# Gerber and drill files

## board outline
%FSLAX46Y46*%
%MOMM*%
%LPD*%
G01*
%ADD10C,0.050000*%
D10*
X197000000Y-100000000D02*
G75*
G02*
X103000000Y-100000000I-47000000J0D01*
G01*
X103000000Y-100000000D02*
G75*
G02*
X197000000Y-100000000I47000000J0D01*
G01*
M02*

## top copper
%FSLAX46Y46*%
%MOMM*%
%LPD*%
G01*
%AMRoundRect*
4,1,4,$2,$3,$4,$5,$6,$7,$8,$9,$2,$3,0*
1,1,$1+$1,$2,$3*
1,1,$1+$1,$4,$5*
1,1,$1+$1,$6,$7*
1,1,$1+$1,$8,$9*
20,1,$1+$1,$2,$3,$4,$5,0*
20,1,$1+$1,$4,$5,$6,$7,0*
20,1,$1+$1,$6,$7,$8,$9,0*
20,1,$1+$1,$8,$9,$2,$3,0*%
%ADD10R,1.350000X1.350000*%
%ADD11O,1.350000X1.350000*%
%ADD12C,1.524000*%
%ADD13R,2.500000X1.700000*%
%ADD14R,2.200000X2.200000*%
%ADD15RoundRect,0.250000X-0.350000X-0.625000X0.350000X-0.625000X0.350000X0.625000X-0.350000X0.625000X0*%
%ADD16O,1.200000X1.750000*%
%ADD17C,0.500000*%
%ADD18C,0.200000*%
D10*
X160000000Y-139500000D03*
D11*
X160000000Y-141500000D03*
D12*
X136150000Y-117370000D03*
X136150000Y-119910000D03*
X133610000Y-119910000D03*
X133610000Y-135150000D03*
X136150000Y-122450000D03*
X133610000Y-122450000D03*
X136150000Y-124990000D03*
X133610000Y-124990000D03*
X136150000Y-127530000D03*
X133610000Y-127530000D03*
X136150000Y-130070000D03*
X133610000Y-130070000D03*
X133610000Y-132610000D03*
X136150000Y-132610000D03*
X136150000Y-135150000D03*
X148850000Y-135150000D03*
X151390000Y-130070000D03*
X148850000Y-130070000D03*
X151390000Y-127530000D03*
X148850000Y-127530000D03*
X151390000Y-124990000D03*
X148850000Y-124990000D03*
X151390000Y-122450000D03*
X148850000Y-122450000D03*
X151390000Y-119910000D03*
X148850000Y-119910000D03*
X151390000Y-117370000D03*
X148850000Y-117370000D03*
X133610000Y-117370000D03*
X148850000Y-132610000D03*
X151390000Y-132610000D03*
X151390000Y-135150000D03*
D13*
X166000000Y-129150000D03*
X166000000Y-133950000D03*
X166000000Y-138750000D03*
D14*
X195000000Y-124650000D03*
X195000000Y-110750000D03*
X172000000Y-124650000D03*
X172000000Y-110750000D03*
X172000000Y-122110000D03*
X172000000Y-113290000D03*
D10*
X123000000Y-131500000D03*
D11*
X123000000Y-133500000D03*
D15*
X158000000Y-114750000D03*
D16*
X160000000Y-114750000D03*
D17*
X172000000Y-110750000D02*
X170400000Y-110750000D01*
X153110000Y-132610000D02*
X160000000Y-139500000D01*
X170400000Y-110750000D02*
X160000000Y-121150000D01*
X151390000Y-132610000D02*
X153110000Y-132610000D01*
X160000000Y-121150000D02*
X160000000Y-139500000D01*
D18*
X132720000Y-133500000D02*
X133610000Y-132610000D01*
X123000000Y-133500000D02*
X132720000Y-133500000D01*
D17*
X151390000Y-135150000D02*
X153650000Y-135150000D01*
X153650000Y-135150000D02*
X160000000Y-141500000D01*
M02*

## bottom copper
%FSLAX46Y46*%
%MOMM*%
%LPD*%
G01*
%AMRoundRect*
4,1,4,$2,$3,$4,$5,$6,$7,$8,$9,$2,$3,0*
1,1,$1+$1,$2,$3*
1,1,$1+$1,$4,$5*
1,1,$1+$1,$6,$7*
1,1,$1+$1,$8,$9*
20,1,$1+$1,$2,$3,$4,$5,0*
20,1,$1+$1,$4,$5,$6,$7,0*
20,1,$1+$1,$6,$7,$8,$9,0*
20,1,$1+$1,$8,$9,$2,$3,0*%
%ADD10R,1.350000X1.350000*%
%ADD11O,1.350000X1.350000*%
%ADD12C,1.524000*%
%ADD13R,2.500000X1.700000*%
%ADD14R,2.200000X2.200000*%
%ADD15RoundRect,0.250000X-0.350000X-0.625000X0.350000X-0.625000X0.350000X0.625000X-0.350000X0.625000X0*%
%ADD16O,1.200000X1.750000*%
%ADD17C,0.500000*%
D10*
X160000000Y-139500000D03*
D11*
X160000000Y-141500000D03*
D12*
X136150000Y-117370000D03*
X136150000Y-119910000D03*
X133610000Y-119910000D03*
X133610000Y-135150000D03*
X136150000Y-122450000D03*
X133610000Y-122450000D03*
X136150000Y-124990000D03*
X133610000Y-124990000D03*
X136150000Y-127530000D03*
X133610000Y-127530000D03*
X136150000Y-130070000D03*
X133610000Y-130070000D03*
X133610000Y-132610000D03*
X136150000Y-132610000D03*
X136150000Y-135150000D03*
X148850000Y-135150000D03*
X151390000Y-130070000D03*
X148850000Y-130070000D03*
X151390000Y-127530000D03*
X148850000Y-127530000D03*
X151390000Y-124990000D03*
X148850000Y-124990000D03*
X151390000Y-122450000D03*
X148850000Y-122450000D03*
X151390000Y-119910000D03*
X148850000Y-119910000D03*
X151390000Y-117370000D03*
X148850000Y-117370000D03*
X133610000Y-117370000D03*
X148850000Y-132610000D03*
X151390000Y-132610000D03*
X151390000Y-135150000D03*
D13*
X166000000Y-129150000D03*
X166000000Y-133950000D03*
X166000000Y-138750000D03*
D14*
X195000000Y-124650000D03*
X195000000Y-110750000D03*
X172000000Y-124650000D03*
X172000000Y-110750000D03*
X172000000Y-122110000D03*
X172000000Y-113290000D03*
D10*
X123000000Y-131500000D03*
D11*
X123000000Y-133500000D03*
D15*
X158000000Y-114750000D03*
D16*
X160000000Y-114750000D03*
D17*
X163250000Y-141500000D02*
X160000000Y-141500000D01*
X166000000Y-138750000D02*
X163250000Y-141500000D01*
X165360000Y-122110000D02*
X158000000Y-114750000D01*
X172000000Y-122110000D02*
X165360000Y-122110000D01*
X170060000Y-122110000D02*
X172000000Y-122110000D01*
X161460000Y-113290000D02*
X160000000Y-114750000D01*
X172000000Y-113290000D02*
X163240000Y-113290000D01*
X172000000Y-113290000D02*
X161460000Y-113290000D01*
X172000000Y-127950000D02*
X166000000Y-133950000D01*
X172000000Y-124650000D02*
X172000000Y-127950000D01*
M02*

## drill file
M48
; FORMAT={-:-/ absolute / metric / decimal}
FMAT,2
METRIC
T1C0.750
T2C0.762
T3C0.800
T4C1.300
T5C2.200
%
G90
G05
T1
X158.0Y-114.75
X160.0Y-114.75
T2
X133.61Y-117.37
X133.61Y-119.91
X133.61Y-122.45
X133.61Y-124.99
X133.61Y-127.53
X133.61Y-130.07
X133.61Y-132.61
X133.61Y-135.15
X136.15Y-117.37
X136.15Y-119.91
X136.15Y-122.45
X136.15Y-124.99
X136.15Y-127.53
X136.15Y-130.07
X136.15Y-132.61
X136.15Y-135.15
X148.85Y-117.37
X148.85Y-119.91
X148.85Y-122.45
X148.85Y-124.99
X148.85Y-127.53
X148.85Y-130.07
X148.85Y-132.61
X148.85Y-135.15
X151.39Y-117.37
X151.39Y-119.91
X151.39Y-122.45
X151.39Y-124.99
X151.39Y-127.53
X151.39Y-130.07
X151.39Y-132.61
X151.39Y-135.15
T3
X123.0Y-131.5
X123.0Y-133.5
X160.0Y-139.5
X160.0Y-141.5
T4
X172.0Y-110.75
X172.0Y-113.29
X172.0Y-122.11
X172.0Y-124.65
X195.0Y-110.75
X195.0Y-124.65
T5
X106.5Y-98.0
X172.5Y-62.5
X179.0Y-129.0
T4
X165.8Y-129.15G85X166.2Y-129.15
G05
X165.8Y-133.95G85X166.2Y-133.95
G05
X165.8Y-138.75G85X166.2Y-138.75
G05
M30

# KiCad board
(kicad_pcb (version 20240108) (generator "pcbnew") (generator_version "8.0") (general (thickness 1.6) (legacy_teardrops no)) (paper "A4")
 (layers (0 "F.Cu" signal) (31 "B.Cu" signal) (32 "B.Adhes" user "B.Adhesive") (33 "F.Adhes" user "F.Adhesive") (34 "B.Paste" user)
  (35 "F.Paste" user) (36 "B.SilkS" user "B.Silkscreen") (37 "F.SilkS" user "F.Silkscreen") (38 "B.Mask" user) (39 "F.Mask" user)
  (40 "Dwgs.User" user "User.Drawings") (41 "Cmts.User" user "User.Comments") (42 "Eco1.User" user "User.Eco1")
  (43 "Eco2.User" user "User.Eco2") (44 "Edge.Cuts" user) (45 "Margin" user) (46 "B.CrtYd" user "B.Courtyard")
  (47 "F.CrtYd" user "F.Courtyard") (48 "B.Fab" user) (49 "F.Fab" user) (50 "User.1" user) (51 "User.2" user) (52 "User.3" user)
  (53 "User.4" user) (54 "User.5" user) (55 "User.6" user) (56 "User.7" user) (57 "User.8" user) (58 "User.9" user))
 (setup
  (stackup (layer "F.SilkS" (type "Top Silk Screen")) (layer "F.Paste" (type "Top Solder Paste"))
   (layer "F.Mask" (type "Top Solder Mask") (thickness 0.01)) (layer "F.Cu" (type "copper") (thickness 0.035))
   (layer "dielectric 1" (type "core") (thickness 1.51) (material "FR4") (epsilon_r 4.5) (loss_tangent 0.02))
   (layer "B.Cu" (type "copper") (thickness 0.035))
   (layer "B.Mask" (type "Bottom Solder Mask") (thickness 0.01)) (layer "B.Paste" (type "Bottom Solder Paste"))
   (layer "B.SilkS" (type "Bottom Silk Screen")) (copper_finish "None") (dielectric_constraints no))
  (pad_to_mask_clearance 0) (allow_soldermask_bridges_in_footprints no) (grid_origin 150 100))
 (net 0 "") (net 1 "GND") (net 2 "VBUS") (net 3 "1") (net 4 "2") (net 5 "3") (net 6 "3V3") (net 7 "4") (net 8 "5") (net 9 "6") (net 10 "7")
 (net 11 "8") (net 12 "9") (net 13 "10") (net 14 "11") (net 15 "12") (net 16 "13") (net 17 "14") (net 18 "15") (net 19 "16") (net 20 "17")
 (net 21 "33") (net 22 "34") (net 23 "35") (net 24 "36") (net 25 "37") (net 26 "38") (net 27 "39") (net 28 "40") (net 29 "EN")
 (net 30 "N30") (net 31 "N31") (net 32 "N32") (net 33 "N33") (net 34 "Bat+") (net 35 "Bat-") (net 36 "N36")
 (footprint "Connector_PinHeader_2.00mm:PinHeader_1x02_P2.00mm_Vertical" (layer "F.Cu") (at 160 139.5)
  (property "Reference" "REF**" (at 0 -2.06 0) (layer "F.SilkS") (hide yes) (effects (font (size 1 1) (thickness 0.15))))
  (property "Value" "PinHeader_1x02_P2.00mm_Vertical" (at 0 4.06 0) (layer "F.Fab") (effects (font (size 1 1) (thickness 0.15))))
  (pad "1" thru_hole rect (at 0 0) (size 1.35 1.35) (drill 0.8) (layers "*.Cu" "*.Mask") (remove_unused_layers no) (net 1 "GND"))
  (pad "2" thru_hole oval (at 0 2) (size 1.35 1.35) (drill 0.8) (layers "*.Cu" "*.Mask") (remove_unused_layers no) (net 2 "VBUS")))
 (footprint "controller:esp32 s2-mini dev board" (layer "F.Cu") (at 142.5 122.45)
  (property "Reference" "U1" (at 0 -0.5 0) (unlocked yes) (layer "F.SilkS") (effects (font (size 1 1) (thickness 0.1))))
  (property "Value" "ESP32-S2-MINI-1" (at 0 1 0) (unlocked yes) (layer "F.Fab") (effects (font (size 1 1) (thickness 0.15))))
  (pad "1" thru_hole circle (at -6.35 -5.08) (size 1.524 1.524) (drill 0.762) (layers "*.Cu" "*.Mask") (remove_unused_layers no) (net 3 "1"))
  (pad "2" thru_hole circle (at -6.35 -2.54) (size 1.524 1.524) (drill 0.762) (layers "*.Cu" "*.Mask") (remove_unused_layers no) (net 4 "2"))
  (pad "3" thru_hole circle (at -8.89 -2.54) (size 1.524 1.524) (drill 0.762) (layers "*.Cu" "*.Mask") (remove_unused_layers no) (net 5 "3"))
  (pad "3V3" thru_hole circle (at -8.89 12.7) (size 1.524 1.524) (drill 0.762) (layers "*.Cu" "*.Mask") (remove_unused_layers no)
   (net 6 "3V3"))
  (pad "4" thru_hole circle (at -6.35 0) (size 1.524 1.524) (drill 0.762) (layers "*.Cu" "*.Mask") (remove_unused_layers no) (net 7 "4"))
  (pad "5" thru_hole circle (at -8.89 0) (size 1.524 1.524) (drill 0.762) (layers "*.Cu" "*.Mask") (remove_unused_layers no) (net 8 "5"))
  (pad "6" thru_hole circle (at -6.35 2.54) (size 1.524 1.524) (drill 0.762) (layers "*.Cu" "*.Mask") (remove_unused_layers no) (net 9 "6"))
  (pad "7" thru_hole circle (at -8.89 2.54) (size 1.524 1.524) (drill 0.762) (layers "*.Cu" "*.Mask") (remove_unused_layers no) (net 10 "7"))
  (pad "8" thru_hole circle (at -6.35 5.08) (size 1.524 1.524) (drill 0.762) (layers "*.Cu" "*.Mask") (remove_unused_layers no) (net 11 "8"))
  (pad "9" thru_hole circle (at -8.89 5.08) (size 1.524 1.524) (drill 0.762) (layers "*.Cu" "*.Mask") (remove_unused_layers no) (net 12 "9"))
  (pad "10" thru_hole circle (at -6.35 7.62) (size 1.524 1.524) (drill 0.762) (layers "*.Cu" "*.Mask") (remove_unused_layers no)
   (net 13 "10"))
  (pad "11" thru_hole circle (at -8.89 7.62) (size 1.524 1.524) (drill 0.762) (layers "*.Cu" "*.Mask") (remove_unused_layers no)
   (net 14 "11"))
  (pad "12" thru_hole circle (at -8.89 10.16) (size 1.524 1.524) (drill 0.762) (layers "*.Cu" "*.Mask") (remove_unused_layers no)
   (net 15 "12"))
  (pad "13" thru_hole circle (at -6.35 10.16) (size 1.524 1.524) (drill 0.762) (layers "*.Cu" "*.Mask") (remove_unused_layers no)
   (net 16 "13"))
  (pad "14" thru_hole circle (at -6.35 12.7) (size 1.524 1.524) (drill 0.762) (layers "*.Cu" "*.Mask") (remove_unused_layers no)
   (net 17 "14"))
  (pad "15" thru_hole circle (at 6.35 12.7) (size 1.524 1.524) (drill 0.762) (layers "*.Cu" "*.Mask") (remove_unused_layers no)
   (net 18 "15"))
  (pad "16" thru_hole circle (at 8.89 7.62) (size 1.524 1.524) (drill 0.762) (layers "*.Cu" "*.Mask") (remove_unused_layers no)
   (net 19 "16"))
  (pad "17" thru_hole circle (at 6.35 7.62) (size 1.524 1.524) (drill 0.762) (layers "*.Cu" "*.Mask") (remove_unused_layers no))
  (pad "18" thru_hole circle (at 8.89 5.08) (size 1.524 1.524) (drill 0.762) (layers "*.Cu" "*.Mask") (remove_unused_layers no))
  (pad "21" thru_hole circle (at 6.35 5.08) (size 1.524 1.524) (drill 0.762) (layers "*.Cu" "*.Mask") (remove_unused_layers no)
   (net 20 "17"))
  (pad "33" thru_hole circle (at 8.89 2.54) (size 1.524 1.524) (drill 0.762) (layers "*.Cu" "*.Mask") (remove_unused_layers no)
   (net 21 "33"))
  (pad "34" thru_hole circle (at 6.35 2.54) (size 1.524 1.524) (drill 0.762) (layers "*.Cu" "*.Mask") (remove_unused_layers no)
   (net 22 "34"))
  (pad "35" thru_hole circle (at 8.89 0) (size 1.524 1.524) (drill 0.762) (layers "*.Cu" "*.Mask") (remove_unused_layers no) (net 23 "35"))
  (pad "36" thru_hole circle (at 6.35 0) (size 1.524 1.524) (drill 0.762) (layers "*.Cu" "*.Mask") (remove_unused_layers no) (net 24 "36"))
  (pad "37" thru_hole circle (at 8.89 -2.54) (size 1.524 1.524) (drill 0.762) (layers "*.Cu" "*.Mask") (remove_unused_layers no)
   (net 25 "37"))
  (pad "38" thru_hole circle (at 6.35 -2.54) (size 1.524 1.524) (drill 0.762) (layers "*.Cu" "*.Mask") (remove_unused_layers no)
   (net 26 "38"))
  (pad "39" thru_hole circle (at 8.89 -5.08) (size 1.524 1.524) (drill 0.762) (layers "*.Cu" "*.Mask") (remove_unused_layers no)
   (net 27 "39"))
  (pad "40" thru_hole circle (at 6.35 -5.08) (size 1.524 1.524) (drill 0.762) (layers "*.Cu" "*.Mask") (remove_unused_layers no)
   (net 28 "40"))
  (pad "EN" thru_hole circle (at -8.89 -5.08) (size 1.524 1.524) (drill 0.762) (layers "*.Cu" "*.Mask") (remove_unused_layers no)
   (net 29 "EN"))
  (pad "GND" thru_hole circle (at 6.35 10.16) (size 1.524 1.524) (drill 0.762) (layers "*.Cu" "*.Mask") (remove_unused_layers no)
   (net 1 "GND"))
  (pad "GND" thru_hole circle (at 8.89 10.16) (size 1.524 1.524) (drill 0.762) (layers "*.Cu" "*.Mask") (remove_unused_layers no)
   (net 1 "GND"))
  (pad "VBUS" thru_hole circle (at 8.89 12.7) (size 1.524 1.524) (drill 0.762) (layers "*.Cu" "*.Mask") (remove_unused_layers no)))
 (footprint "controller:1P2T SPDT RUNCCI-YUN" (layer "F.Cu") (at 166 133.95)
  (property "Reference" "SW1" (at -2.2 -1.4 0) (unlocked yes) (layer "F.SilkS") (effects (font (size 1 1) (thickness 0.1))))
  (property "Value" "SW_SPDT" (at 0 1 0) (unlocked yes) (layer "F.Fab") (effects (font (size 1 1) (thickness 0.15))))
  (pad "1" thru_hole rect (at 0 -4.8) (size 2.5 1.7) (drill oval 1.7 1.3) (layers "*.Cu" "*.Mask") (remove_unused_layers no) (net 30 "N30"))
  (pad "2" thru_hole rect (at 0 0) (size 2.5 1.7) (drill oval 1.7 1.3) (layers "*.Cu" "*.Mask") (remove_unused_layers no) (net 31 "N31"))
  (pad "3" thru_hole rect (at 0 4.8) (size 2.5 1.7) (drill oval 1.7 1.3) (layers "*.Cu" "*.Mask") (remove_unused_layers no) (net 2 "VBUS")))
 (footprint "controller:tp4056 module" (layer "F.Cu") (at 195 124.65 180)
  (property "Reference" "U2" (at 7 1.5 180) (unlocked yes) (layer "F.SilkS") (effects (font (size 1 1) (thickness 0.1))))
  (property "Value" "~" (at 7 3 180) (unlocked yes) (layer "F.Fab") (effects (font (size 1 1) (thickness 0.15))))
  (pad "1" thru_hole rect (at 0 0 180) (size 2.2 2.2) (drill 1.3) (layers "*.Cu" "*.Mask") (remove_unused_layers no) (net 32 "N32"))
  (pad "2" thru_hole rect (at 0 13.9 180) (size 2.2 2.2) (drill 1.3) (layers "*.Cu" "*.Mask") (remove_unused_layers no) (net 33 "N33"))
  (pad "3" thru_hole rect (at 23 0 180) (size 2.2 2.2) (drill 1.3) (layers "*.Cu" "*.Mask") (remove_unused_layers no) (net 31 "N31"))
  (pad "4" thru_hole rect (at 23 13.9 180) (size 2.2 2.2) (drill 1.3) (layers "*.Cu" "*.Mask") (remove_unused_layers no) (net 1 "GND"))
  (pad "5" thru_hole rect (at 23 2.54 180) (size 2.2 2.2) (drill 1.3) (layers "*.Cu" "*.Mask") (remove_unused_layers no) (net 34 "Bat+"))
  (pad "6" thru_hole rect (at 23 11.36 180) (size 2.2 2.2) (drill 1.3) (layers "*.Cu" "*.Mask") (remove_unused_layers no) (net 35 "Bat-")))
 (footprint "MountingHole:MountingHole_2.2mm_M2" (layer "F.Cu") (at 172.5 62.5)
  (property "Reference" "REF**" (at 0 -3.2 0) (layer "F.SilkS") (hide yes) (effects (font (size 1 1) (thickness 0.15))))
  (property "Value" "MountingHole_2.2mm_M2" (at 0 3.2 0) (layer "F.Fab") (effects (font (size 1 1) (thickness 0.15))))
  (pad "" np_thru_hole circle (at 0 0) (size 2.2 2.2) (drill 2.2) (layers "*.Cu" "*.Mask")))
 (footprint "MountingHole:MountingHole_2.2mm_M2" (layer "F.Cu") (at 179 129)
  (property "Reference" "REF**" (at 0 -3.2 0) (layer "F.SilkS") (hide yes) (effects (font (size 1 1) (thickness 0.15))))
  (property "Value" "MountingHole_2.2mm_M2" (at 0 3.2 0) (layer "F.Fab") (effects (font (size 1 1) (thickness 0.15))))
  (pad "" np_thru_hole circle (at 0 0) (size 2.2 2.2) (drill 2.2) (layers "F&B.Cu" "*.Mask")))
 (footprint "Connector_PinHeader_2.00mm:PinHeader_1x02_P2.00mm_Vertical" (layer "F.Cu") (at 123 131.5)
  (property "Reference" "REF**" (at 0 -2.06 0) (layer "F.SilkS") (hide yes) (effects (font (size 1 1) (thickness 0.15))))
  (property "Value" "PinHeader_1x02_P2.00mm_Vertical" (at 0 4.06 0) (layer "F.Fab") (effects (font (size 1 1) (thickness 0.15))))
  (pad "1" thru_hole rect (at 0 0) (size 1.35 1.35) (drill 0.8) (layers "*.Cu" "*.Mask") (remove_unused_layers no) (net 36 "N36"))
  (pad "2" thru_hole oval (at 0 2) (size 1.35 1.35) (drill 0.8) (layers "*.Cu" "*.Mask") (remove_unused_layers no) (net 15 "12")))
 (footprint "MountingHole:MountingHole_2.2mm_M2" (layer "F.Cu") (at 106.5 98)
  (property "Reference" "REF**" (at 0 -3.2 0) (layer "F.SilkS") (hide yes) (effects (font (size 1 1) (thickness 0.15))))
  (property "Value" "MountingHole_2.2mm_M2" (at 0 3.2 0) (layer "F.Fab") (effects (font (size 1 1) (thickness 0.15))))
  (pad "" np_thru_hole circle (at 0 0) (size 2.2 2.2) (drill 2.2) (layers "F&B.Cu" "*.Mask")))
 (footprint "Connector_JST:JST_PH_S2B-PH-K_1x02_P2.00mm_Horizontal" (layer "B.Cu") (at 158 114.75)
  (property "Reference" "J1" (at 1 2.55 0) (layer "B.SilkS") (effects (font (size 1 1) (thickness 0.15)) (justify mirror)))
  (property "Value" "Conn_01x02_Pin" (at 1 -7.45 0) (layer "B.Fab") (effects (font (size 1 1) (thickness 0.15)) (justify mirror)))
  (pad "1" thru_hole roundrect (at 0 0) (size 1.2 1.75) (drill 0.75) (layers "*.Cu" "*.Mask") (remove_unused_layers no)
   (roundrect_rratio 0.208333) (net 34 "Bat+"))
  (pad "2" thru_hole oval (at 2 0) (size 1.2 1.75) (drill 0.75) (layers "*.Cu" "*.Mask") (remove_unused_layers no) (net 35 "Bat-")))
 (gr_circle (center 150 100) (end 197 100) (stroke (width 0.05) (type default)) (fill none) (layer "Edge.Cuts"))
 (segment (start 172 110.75) (end 170.4 110.75) (width 0.5) (layer "F.Cu") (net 1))
 (segment (start 153.11 132.61) (end 160 139.5) (width 0.5) (layer "F.Cu") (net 1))
 (segment (start 170.4 110.75) (end 160 121.15) (width 0.5) (layer "F.Cu") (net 1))
 (segment (start 151.39 132.61) (end 153.11 132.61) (width 0.5) (layer "F.Cu") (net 1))
 (segment (start 160 121.15) (end 160 139.5) (width 0.5) (layer "F.Cu") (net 1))
 (segment (start 132.72 133.5) (end 133.61 132.61) (width 0.2) (layer "F.Cu") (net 15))
 (segment (start 123 133.5) (end 132.72 133.5) (width 0.2) (layer "F.Cu") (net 15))
 (segment (start 151.39 135.15) (end 153.65 135.15) (width 0.5) (layer "F.Cu") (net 2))
 (segment (start 153.65 135.15) (end 160 141.5) (width 0.5) (layer "F.Cu") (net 2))
 (segment (start 163.25 141.5) (end 160 141.5) (width 0.5) (layer "B.Cu") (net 2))
 (segment (start 166 138.75) (end 163.25 141.5) (width 0.5) (layer "B.Cu") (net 2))
 (segment (start 165.36 122.11) (end 158 114.75) (width 0.5) (layer "B.Cu") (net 34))
 (segment (start 172 122.11) (end 165.36 122.11) (width 0.5) (layer "B.Cu") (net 34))
 (segment (start 170.06 122.11) (end 172 122.11) (width 0.5) (layer "B.Cu") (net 34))
 (segment (start 161.46 113.29) (end 160 114.75) (width 0.5) (layer "B.Cu") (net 35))
 (segment (start 172 113.29) (end 163.24 113.29) (width 0.5) (layer "B.Cu") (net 35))
 (segment (start 172 113.29) (end 161.46 113.29) (width 0.5) (layer "B.Cu") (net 35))
 (segment (start 172 127.95) (end 166 133.95) (width 0.5) (layer "B.Cu") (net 31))
 (segment (start 172 124.65) (end 172 127.95) (width 0.5) (layer "B.Cu") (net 31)))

